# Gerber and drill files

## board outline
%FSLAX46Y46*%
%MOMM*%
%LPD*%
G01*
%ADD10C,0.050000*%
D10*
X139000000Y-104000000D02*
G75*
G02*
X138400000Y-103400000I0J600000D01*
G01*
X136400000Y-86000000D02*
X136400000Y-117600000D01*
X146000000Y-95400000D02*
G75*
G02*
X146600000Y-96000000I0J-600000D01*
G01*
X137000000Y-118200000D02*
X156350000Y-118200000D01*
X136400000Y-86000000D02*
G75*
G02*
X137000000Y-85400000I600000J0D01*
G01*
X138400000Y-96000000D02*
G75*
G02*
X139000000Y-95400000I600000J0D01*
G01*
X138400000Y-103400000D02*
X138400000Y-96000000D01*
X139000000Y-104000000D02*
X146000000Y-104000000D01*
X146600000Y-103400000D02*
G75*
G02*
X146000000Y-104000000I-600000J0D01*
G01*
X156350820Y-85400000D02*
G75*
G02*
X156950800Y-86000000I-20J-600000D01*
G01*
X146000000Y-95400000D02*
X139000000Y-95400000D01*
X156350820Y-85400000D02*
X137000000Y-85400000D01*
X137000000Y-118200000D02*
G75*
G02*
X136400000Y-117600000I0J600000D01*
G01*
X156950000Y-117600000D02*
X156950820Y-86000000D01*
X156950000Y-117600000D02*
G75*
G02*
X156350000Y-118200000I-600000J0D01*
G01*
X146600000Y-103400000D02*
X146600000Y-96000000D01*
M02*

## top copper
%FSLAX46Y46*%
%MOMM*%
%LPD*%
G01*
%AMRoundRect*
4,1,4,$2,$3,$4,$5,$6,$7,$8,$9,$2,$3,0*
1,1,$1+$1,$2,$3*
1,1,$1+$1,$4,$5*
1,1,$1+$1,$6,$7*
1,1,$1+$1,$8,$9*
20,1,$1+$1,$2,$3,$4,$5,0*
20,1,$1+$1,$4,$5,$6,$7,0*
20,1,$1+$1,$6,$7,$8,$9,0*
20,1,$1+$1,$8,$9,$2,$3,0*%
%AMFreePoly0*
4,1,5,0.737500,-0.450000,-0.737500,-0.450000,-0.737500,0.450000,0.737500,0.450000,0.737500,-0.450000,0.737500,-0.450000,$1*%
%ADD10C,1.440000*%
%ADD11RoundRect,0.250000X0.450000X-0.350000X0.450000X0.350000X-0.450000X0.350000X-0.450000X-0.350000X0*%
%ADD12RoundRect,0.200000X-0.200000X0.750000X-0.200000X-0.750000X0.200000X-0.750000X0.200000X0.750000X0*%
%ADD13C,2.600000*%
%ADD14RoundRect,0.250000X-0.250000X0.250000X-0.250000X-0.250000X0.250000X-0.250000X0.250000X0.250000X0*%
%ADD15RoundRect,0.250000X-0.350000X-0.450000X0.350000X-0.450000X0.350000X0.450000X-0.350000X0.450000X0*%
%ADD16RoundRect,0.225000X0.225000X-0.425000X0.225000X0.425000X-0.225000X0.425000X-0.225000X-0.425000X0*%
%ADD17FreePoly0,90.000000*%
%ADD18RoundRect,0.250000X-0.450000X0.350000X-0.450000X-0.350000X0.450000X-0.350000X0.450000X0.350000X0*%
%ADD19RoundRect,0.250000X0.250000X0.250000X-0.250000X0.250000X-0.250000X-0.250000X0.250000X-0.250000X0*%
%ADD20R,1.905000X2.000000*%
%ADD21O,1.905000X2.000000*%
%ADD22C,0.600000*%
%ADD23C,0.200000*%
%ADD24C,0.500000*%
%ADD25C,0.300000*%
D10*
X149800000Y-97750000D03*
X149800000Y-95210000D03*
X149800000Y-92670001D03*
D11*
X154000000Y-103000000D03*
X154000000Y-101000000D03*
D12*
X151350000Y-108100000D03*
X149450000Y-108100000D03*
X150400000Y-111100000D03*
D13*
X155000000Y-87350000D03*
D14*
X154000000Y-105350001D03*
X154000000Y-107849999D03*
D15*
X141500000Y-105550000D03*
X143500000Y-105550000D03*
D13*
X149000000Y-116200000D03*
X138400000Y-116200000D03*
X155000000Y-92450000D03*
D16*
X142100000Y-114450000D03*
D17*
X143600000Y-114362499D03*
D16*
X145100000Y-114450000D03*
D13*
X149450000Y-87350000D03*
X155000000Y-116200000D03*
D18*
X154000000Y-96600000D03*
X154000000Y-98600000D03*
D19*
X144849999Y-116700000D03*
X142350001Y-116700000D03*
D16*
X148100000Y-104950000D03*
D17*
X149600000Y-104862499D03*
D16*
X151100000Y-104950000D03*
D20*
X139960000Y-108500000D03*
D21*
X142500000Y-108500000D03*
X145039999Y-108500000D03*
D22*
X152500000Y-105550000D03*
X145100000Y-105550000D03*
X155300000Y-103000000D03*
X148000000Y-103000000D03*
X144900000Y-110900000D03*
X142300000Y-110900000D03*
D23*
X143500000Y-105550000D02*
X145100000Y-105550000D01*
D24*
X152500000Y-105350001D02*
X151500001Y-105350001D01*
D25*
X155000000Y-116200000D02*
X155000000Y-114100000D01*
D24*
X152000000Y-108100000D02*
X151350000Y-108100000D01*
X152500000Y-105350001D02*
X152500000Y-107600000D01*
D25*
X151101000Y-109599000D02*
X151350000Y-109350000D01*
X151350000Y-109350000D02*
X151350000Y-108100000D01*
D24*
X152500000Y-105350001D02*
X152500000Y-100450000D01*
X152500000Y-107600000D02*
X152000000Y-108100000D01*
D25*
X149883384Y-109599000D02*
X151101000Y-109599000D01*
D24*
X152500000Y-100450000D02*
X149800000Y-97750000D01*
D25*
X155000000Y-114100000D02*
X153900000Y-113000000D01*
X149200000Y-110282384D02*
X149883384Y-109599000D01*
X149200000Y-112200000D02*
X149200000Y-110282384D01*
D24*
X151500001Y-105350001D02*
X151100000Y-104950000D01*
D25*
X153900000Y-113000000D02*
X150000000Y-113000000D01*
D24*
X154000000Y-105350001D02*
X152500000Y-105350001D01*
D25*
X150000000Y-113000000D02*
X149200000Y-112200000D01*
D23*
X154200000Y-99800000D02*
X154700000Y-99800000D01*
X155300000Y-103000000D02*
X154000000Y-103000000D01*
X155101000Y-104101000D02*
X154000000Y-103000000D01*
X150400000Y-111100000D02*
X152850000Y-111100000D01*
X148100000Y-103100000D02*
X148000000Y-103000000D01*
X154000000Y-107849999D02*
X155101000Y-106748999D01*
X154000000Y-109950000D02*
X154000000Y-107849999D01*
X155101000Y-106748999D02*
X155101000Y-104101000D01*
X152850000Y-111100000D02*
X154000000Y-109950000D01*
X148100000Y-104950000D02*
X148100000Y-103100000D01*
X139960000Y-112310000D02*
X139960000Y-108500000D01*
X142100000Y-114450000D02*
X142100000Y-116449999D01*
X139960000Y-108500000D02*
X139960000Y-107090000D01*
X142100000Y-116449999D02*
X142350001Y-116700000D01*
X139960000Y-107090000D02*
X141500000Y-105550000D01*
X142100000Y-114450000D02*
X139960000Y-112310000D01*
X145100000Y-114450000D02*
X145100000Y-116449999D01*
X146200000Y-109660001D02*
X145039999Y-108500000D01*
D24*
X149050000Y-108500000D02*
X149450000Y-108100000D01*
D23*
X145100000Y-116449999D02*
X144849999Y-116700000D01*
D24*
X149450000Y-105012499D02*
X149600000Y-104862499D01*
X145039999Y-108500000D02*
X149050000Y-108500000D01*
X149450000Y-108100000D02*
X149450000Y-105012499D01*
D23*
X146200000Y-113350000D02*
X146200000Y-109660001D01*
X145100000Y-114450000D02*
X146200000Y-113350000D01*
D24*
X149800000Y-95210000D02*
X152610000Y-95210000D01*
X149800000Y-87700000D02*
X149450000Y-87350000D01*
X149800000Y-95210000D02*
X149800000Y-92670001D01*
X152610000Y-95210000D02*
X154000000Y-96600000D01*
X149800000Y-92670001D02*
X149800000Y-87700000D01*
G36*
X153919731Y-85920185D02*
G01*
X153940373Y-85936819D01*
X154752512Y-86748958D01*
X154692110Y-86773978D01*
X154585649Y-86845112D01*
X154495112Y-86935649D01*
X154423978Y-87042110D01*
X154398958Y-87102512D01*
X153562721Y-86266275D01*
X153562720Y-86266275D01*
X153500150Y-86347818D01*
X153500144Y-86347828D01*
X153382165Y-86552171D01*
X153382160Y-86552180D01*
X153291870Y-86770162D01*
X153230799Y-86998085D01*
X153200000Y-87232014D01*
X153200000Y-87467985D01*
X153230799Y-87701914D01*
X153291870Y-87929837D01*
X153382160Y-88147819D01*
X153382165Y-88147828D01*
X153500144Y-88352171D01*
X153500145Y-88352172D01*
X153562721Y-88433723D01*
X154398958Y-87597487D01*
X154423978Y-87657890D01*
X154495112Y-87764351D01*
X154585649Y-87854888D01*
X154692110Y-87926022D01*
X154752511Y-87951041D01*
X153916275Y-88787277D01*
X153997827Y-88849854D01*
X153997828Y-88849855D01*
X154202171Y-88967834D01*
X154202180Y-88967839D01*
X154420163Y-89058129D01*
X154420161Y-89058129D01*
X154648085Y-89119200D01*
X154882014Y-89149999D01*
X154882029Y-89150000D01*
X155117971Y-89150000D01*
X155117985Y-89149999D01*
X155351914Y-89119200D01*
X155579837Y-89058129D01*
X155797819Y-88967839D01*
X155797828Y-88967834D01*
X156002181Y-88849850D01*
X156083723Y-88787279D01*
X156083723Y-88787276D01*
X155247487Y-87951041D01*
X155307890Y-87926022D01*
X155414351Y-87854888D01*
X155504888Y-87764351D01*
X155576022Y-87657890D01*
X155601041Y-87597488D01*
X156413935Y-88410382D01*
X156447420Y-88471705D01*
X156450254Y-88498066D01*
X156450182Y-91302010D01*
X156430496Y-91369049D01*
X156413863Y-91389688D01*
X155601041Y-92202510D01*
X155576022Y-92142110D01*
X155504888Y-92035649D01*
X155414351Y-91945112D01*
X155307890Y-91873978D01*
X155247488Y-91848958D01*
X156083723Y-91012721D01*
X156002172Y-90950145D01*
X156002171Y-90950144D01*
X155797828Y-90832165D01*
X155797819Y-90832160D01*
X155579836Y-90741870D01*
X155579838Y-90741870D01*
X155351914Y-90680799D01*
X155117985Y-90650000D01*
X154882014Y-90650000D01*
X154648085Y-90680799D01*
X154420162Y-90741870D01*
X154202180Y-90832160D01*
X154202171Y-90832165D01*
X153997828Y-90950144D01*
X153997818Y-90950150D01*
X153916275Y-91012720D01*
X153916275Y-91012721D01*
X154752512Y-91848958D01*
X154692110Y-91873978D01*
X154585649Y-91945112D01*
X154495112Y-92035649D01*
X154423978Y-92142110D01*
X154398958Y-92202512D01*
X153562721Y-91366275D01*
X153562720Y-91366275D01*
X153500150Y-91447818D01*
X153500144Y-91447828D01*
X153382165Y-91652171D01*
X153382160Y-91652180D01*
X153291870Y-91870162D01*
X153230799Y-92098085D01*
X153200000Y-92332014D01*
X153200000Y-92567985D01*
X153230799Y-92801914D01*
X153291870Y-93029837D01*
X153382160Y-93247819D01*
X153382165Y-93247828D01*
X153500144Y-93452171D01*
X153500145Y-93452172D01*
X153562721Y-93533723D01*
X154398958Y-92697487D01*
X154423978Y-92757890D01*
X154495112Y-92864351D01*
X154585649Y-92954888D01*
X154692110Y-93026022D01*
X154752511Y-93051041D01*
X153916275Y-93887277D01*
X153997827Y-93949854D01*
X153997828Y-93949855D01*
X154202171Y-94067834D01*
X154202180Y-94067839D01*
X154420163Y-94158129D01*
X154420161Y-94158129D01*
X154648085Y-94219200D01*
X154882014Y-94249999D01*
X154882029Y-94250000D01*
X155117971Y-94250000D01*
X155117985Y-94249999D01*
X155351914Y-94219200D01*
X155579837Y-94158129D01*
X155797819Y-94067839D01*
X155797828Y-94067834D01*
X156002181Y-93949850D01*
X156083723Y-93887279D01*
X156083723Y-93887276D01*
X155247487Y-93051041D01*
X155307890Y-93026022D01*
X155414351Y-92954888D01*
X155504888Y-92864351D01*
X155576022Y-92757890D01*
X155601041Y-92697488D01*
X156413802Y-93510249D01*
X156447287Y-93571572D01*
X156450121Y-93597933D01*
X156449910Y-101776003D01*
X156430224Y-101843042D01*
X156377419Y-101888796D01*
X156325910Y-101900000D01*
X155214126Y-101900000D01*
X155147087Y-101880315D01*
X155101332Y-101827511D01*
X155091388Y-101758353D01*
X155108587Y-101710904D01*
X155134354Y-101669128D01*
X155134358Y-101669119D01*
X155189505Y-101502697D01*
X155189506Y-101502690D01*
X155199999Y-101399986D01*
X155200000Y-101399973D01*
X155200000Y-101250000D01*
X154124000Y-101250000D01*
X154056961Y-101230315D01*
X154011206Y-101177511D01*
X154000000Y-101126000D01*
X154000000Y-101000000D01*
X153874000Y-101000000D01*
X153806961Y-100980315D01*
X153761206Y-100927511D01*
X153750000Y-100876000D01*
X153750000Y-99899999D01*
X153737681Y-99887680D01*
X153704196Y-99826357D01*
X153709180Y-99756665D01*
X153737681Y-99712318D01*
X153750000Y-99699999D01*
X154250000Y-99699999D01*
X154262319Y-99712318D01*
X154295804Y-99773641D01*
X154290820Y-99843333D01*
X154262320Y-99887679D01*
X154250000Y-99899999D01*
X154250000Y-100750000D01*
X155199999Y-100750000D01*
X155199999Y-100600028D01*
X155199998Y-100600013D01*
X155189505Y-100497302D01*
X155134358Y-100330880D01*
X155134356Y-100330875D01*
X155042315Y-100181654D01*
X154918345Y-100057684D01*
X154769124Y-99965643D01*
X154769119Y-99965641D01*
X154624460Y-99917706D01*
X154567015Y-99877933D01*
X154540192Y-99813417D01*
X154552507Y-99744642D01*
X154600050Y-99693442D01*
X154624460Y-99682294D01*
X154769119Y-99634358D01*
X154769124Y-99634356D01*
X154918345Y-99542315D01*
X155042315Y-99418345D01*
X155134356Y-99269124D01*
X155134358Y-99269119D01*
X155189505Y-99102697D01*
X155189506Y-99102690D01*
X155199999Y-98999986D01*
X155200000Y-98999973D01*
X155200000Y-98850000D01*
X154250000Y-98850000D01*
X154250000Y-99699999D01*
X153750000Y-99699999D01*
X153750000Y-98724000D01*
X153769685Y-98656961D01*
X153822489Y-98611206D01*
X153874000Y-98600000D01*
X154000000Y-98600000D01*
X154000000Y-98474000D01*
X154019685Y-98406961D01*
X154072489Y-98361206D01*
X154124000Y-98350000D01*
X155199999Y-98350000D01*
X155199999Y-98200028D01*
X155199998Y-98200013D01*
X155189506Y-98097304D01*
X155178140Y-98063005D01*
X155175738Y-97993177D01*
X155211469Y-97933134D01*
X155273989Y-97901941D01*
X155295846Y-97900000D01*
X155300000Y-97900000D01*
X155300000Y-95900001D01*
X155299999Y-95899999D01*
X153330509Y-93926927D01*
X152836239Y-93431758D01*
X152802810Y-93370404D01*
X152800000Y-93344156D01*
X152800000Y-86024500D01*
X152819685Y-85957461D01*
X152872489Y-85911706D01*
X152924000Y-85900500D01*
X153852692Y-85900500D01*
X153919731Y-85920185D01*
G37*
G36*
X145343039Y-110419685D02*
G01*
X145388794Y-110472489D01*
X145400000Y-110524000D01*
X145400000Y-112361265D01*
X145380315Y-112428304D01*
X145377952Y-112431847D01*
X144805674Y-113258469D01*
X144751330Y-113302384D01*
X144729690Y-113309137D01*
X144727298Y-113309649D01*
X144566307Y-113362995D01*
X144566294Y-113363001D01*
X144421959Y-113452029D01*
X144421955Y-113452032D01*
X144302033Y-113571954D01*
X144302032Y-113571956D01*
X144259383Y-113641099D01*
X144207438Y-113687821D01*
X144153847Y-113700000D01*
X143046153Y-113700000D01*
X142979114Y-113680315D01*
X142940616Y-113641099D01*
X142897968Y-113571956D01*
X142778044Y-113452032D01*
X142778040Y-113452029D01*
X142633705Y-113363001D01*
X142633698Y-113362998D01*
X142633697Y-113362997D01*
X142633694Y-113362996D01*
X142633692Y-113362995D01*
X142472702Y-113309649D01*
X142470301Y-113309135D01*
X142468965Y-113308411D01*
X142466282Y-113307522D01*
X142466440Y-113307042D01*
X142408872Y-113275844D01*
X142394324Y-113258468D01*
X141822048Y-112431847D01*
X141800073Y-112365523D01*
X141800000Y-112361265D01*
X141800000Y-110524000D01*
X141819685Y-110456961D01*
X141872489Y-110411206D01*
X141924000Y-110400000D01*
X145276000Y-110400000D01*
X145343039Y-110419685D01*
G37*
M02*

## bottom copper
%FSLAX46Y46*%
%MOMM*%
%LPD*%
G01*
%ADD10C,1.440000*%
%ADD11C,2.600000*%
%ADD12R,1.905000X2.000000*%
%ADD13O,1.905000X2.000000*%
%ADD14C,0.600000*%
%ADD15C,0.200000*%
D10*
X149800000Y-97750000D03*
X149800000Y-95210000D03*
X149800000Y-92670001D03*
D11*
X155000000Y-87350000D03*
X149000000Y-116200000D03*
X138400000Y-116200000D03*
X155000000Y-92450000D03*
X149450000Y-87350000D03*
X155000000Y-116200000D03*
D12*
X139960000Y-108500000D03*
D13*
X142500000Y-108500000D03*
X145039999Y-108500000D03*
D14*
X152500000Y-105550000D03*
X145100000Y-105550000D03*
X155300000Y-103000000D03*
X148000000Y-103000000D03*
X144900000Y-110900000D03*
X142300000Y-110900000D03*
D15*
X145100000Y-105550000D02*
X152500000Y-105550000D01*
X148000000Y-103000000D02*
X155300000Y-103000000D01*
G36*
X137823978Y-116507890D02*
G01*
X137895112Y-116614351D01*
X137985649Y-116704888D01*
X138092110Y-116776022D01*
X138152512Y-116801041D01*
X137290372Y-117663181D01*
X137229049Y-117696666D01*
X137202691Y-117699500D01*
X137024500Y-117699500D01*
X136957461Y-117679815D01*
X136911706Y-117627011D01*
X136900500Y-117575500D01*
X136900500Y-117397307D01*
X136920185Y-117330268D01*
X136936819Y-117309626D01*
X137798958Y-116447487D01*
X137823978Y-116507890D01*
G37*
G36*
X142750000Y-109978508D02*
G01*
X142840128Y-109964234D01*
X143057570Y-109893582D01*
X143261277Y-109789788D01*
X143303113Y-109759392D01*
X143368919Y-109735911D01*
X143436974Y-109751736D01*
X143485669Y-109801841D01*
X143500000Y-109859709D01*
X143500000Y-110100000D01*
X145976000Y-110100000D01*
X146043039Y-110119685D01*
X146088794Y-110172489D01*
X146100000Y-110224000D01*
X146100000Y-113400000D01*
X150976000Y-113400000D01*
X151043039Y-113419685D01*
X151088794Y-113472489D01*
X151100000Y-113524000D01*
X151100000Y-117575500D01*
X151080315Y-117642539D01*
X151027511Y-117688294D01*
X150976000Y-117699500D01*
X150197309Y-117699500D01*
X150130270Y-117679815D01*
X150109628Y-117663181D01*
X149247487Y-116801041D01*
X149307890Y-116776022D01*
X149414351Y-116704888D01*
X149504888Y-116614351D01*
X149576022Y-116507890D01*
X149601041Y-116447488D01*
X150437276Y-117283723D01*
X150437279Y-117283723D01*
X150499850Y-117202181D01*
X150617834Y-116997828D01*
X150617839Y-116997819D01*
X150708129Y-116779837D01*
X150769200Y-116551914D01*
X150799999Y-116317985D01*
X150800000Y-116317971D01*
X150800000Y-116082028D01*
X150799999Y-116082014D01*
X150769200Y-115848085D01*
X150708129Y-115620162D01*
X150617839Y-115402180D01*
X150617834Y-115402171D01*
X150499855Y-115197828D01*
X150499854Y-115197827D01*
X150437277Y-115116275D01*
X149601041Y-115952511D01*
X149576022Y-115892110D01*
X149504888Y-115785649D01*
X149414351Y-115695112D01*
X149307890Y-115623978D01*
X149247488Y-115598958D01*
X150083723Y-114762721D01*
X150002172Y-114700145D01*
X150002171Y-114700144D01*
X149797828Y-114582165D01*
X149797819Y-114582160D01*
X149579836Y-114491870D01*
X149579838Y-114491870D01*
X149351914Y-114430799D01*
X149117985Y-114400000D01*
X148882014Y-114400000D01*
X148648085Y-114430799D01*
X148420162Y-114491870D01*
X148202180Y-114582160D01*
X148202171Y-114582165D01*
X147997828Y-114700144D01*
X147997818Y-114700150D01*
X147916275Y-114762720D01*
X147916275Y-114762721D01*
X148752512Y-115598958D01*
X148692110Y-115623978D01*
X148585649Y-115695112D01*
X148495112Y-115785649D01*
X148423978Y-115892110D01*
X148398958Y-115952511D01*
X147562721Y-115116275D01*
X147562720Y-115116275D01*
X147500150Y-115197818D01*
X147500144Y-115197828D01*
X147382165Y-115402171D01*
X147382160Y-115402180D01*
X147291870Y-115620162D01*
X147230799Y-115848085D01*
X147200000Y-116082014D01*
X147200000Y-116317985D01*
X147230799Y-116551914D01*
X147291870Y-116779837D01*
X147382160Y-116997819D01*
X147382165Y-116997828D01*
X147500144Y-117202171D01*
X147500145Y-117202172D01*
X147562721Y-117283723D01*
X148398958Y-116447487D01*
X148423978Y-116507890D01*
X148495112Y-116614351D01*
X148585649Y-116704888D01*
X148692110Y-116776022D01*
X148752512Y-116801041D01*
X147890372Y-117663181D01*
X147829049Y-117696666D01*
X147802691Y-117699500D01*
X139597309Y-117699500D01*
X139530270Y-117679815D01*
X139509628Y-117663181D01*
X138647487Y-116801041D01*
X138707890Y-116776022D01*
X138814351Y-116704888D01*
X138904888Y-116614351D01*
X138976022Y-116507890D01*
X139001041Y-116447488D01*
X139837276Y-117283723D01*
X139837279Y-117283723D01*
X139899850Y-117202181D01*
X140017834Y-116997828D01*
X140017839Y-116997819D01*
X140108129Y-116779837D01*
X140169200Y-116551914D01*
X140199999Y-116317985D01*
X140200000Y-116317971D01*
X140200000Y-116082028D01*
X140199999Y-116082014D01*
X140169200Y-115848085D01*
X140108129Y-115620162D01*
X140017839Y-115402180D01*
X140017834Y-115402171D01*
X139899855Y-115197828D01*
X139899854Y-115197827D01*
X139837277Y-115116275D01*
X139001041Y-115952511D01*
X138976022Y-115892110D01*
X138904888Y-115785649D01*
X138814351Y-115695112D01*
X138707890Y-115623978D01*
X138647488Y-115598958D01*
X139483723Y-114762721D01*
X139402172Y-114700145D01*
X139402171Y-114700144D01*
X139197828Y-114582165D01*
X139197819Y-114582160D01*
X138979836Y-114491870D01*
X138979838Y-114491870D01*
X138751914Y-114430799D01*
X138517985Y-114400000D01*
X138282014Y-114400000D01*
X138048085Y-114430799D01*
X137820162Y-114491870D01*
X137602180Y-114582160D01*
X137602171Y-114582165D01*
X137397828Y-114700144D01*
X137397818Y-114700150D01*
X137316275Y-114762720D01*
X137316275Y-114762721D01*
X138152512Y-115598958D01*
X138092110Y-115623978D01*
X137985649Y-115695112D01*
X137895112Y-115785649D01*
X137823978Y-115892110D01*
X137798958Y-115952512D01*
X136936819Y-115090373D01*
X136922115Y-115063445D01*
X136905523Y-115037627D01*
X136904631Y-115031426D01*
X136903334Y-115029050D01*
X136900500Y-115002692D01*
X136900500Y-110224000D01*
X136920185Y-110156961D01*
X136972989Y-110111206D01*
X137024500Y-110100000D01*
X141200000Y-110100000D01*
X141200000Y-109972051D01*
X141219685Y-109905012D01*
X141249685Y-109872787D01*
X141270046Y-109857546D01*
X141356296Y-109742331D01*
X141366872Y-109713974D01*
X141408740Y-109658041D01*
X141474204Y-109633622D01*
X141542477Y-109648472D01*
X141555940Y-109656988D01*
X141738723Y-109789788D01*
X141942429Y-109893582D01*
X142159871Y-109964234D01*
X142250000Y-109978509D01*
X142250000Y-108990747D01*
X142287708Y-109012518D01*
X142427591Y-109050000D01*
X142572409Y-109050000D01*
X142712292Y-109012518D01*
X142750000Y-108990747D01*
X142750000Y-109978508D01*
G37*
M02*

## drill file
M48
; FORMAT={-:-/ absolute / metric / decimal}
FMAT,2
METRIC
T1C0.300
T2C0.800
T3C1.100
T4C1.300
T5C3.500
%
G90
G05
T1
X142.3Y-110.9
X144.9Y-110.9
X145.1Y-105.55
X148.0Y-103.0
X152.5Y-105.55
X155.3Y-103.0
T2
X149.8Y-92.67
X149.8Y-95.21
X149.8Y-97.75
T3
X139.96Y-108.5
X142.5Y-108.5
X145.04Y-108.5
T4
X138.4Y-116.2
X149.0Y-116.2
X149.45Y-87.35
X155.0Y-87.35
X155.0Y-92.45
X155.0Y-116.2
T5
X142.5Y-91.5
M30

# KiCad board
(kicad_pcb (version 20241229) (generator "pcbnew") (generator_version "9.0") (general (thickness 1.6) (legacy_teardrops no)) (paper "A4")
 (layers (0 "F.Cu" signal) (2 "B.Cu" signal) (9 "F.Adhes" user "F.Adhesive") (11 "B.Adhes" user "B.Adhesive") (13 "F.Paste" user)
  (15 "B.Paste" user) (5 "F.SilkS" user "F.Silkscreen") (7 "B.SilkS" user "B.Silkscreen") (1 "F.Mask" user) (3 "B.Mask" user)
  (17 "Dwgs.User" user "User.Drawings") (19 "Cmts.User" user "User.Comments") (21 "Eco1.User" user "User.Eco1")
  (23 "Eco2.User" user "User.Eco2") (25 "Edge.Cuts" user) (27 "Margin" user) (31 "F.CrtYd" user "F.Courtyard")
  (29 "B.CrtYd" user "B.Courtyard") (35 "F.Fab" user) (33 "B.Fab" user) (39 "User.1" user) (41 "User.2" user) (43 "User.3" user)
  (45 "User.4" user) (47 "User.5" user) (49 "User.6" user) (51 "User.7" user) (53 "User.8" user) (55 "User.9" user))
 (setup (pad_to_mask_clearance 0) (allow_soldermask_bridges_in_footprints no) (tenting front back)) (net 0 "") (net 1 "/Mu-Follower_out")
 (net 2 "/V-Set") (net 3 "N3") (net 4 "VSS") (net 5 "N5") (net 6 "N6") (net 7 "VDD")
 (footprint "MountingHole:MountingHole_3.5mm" (layer "F.Cu") (at 142.5 91.5)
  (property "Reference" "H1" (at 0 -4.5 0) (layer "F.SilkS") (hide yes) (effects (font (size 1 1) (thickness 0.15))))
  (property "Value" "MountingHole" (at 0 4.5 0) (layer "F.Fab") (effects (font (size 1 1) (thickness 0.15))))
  (pad "" np_thru_hole circle (at 0 0) (size 3.5 3.5) (drill 3.5) (layers "*.Cu" "*.Mask")))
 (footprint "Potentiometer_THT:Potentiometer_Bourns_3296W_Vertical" (layer "F.Cu") (at 149.8 97.75 -90)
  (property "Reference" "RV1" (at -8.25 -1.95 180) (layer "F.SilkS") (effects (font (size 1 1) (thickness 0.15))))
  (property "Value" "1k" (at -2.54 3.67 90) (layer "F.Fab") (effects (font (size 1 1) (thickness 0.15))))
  (pad "1" thru_hole circle (at 0 0 270) (size 1.44 1.44) (drill 0.8) (layers "*.Cu" "*.Mask") (remove_unused_layers no)
   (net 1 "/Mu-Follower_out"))
  (pad "2" thru_hole circle (at -2.54 0 270) (size 1.44 1.44) (drill 0.8) (layers "*.Cu" "*.Mask") (remove_unused_layers no)
   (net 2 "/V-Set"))
  (pad "3" thru_hole circle (at -5.079999 0 270) (size 1.44 1.44) (drill 0.8) (layers "*.Cu" "*.Mask") (remove_unused_layers no)
   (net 2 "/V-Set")))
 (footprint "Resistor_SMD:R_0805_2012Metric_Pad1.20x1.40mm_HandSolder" (layer "F.Cu") (at 154 102 90)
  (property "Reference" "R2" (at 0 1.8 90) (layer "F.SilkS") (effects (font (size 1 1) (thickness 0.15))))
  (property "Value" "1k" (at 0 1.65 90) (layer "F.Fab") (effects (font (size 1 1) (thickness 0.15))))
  (pad "1" smd roundrect (at -1 0 90) (size 1.2 1.4) (layers "F.Cu" "F.Mask" "F.Paste") (roundrect_rratio 0.208333) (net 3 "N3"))
  (pad "2" smd roundrect (at 1 0 90) (size 1.2 1.4) (layers "F.Cu" "F.Mask" "F.Paste") (roundrect_rratio 0.208333) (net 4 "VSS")))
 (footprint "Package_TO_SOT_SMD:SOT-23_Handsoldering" (layer "F.Cu") (at 150.4 109.6 -90)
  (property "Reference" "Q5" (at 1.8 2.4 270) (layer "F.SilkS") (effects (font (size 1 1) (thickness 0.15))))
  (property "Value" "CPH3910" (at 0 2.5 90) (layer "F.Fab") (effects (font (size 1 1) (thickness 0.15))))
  (pad "1" smd roundrect (at -1.5 -0.95 270) (size 1.9 0.8) (layers "F.Cu" "F.Mask" "F.Paste") (roundrect_rratio 0.25)
   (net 1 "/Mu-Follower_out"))
  (pad "2" smd roundrect (at -1.5 0.95 270) (size 1.9 0.8) (layers "F.Cu" "F.Mask" "F.Paste") (roundrect_rratio 0.25) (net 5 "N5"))
  (pad "3" smd roundrect (at 1.5 0 270) (size 1.9 0.8) (layers "F.Cu" "F.Mask" "F.Paste") (roundrect_rratio 0.25) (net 3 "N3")))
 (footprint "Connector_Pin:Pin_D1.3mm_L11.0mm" (layer "F.Cu") (at 155 87.35 180)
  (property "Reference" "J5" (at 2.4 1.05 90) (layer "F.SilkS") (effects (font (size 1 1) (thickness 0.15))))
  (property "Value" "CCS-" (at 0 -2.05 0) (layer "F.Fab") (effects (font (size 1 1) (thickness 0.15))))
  (pad "1" thru_hole circle (at 0 0 180) (size 2.6 2.6) (drill 1.3) (layers "*.Cu" "*.Mask") (remove_unused_layers no) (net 4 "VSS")))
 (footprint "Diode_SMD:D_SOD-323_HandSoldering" (layer "F.Cu") (at 154 106.6 -90)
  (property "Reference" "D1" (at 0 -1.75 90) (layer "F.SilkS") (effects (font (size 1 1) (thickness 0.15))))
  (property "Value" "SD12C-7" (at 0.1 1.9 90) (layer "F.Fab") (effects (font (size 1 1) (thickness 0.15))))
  (pad "1" smd roundrect (at -1.249999 0 270) (size 1 1) (layers "F.Cu" "F.Mask" "F.Paste") (roundrect_rratio 0.25)
   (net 1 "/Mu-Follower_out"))
  (pad "2" smd roundrect (at 1.249999 0 270) (size 1 1) (layers "F.Cu" "F.Mask" "F.Paste") (roundrect_rratio 0.25) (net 3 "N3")))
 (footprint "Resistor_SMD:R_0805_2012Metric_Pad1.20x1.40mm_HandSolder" (layer "F.Cu") (at 142.5 105.55)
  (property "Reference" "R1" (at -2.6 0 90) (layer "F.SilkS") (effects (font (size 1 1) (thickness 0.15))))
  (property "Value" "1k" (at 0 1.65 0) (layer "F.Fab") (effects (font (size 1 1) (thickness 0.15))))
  (pad "1" smd roundrect (at -1 0) (size 1.2 1.4) (layers "F.Cu" "F.Mask" "F.Paste") (roundrect_rratio 0.208333) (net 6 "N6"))
  (pad "2" smd roundrect (at 1 0) (size 1.2 1.4) (layers "F.Cu" "F.Mask" "F.Paste") (roundrect_rratio 0.208333) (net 1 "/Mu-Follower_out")))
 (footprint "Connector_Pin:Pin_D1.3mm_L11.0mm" (layer "F.Cu") (at 149 116.2)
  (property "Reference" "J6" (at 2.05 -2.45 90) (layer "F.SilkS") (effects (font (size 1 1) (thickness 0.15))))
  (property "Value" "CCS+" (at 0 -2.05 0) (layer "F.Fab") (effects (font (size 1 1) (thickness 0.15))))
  (pad "1" thru_hole circle (at 0 0) (size 2.6 2.6) (drill 1.3) (layers "*.Cu" "*.Mask") (remove_unused_layers no) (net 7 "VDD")))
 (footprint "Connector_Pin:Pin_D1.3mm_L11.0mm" (layer "F.Cu") (at 138.4 116.2)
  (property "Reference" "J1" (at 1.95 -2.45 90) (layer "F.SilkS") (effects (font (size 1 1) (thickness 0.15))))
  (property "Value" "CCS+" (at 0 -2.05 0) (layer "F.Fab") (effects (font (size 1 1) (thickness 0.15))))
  (pad "1" thru_hole circle (at 0 0) (size 2.6 2.6) (drill 1.3) (layers "*.Cu" "*.Mask") (remove_unused_layers no) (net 7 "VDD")))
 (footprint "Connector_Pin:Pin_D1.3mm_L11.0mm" (layer "F.Cu") (at 155 92.45 180)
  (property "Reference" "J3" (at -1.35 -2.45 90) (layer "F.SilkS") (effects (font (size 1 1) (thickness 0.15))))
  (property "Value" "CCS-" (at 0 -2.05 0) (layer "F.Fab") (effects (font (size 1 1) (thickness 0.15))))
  (pad "1" thru_hole circle (at 0 0 180) (size 2.6 2.6) (drill 1.3) (layers "*.Cu" "*.Mask") (remove_unused_layers no) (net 4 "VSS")))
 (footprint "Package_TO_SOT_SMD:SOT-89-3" (layer "F.Cu") (at 143.6 112.5 90)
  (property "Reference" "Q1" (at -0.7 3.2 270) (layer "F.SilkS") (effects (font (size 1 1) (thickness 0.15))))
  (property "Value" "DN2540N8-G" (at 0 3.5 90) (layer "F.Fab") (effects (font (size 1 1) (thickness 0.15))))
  (pad "1" smd roundrect (at -1.95 -1.5 90) (size 1.3 0.9) (layers "F.Cu" "F.Mask" "F.Paste") (roundrect_rratio 0.25) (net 6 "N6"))
  (pad "2" smd custom (at -1.862499 0 90) (size 1.475 0.9) (layers "F.Cu" "F.Mask" "F.Paste") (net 7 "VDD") (zone_connect 2)
   (thermal_bridge_angle 45) (options (clearance outline) (anchor rect)) (primitives))
  (pad "3" smd roundrect (at -1.95 1.5 90) (size 1.3 0.9) (layers "F.Cu" "F.Mask" "F.Paste") (roundrect_rratio 0.25) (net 5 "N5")))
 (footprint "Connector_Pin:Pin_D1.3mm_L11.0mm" (layer "F.Cu") (at 149.45 87.35 180)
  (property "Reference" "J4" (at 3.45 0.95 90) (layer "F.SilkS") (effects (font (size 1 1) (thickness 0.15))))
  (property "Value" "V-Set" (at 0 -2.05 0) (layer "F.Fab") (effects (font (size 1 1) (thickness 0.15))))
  (pad "1" thru_hole circle (at 0 0 180) (size 2.6 2.6) (drill 1.3) (layers "*.Cu" "*.Mask") (remove_unused_layers no) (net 2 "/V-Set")))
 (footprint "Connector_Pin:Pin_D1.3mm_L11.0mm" (layer "F.Cu") (at 155 116.2)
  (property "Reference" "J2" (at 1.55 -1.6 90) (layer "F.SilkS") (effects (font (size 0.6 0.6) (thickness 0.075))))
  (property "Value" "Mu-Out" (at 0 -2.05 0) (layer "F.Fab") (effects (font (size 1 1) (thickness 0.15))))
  (pad "1" thru_hole circle (at 0 0) (size 2.6 2.6) (drill 1.3) (layers "*.Cu" "*.Mask") (remove_unused_layers no)
   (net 1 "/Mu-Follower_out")))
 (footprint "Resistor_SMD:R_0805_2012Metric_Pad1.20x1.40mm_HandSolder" (layer "F.Cu") (at 154 97.6 -90)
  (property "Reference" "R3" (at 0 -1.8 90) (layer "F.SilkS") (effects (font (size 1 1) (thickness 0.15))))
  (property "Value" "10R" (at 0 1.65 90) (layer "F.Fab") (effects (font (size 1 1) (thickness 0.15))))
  (pad "1" smd roundrect (at -1 0 270) (size 1.2 1.4) (layers "F.Cu" "F.Mask" "F.Paste") (roundrect_rratio 0.208333) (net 2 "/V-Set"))
  (pad "2" smd roundrect (at 1 0 270) (size 1.2 1.4) (layers "F.Cu" "F.Mask" "F.Paste") (roundrect_rratio 0.208333) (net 4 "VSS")))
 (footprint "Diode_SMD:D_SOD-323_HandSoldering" (layer "F.Cu") (at 143.6 116.7 180)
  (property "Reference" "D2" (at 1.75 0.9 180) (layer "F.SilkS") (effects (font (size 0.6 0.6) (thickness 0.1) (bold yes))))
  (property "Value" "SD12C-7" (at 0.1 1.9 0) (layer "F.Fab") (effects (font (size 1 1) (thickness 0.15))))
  (pad "1" smd roundrect (at -1.249999 0 180) (size 1 1) (layers "F.Cu" "F.Mask" "F.Paste") (roundrect_rratio 0.25) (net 5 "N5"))
  (pad "2" smd roundrect (at 1.249999 0 180) (size 1 1) (layers "F.Cu" "F.Mask" "F.Paste") (roundrect_rratio 0.25) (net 6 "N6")))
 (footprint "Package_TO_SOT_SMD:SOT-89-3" (layer "F.Cu") (at 149.6 103 90)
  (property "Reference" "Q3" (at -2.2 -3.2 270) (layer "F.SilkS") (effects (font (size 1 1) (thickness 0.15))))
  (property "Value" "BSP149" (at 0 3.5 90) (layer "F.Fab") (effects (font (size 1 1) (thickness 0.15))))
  (pad "1" smd roundrect (at -1.95 -1.5 90) (size 1.3 0.9) (layers "F.Cu" "F.Mask" "F.Paste") (roundrect_rratio 0.25) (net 3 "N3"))
  (pad "2" smd custom (at -1.862499 0 90) (size 1.475 0.9) (layers "F.Cu" "F.Mask" "F.Paste") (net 5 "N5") (zone_connect 2)
   (thermal_bridge_angle 45) (options (clearance outline) (anchor rect)) (primitives))
  (pad "3" smd roundrect (at -1.95 1.5 90) (size 1.3 0.9) (layers "F.Cu" "F.Mask" "F.Paste") (roundrect_rratio 0.25)
   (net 1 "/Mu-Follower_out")))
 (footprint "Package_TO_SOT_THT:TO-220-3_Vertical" (layer "B.Cu") (at 139.96 108.5)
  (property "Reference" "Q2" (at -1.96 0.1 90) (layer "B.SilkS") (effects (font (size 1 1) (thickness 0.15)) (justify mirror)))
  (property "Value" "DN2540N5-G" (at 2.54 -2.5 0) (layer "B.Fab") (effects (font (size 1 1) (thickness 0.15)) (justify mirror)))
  (pad "1" thru_hole rect (at 0 0) (size 1.905 2) (drill 1.1) (layers "*.Cu" "*.Mask") (remove_unused_layers no) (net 6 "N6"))
  (pad "2" thru_hole oval (at 2.54 0) (size 1.905 2) (drill 1.1) (layers "*.Cu" "*.Mask") (remove_unused_layers no) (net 7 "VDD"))
  (pad "3" thru_hole oval (at 5.079999 0) (size 1.905 2) (drill 1.1) (layers "*.Cu" "*.Mask") (remove_unused_layers no) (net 5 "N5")))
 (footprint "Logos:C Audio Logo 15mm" (layer "B.Cu") (at 152 111.6)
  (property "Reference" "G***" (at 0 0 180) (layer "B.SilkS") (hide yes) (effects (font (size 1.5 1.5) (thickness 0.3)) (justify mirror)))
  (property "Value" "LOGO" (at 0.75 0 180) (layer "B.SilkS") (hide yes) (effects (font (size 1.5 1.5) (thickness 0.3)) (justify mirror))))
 (gr_arc (start 139 104) (mid 138.575736 103.824264) (end 138.4 103.4) (stroke (width 0.05) (type default)) (layer "Edge.Cuts"))
 (gr_line (start 136.4 86) (end 136.4 117.6) (stroke (width 0.05) (type default)) (layer "Edge.Cuts"))
 (gr_arc (start 146 95.4) (mid 146.424264 95.575736) (end 146.6 96) (stroke (width 0.05) (type default)) (layer "Edge.Cuts"))
 (gr_line (start 137 118.2) (end 156.35 118.2) (stroke (width 0.05) (type default)) (layer "Edge.Cuts"))
 (gr_arc (start 136.4 86) (mid 136.575736 85.575736) (end 137 85.4) (stroke (width 0.05) (type default)) (layer "Edge.Cuts"))
 (gr_arc (start 138.4 96) (mid 138.575736 95.575736) (end 139 95.4) (stroke (width 0.05) (type default)) (layer "Edge.Cuts"))
 (gr_line (start 138.4 103.4) (end 138.4 96) (stroke (width 0.05) (type default)) (layer "Edge.Cuts"))
 (gr_line (start 139 104) (end 146 104) (stroke (width 0.05) (type default)) (layer "Edge.Cuts"))
 (gr_arc (start 146.6 103.4) (mid 146.424264 103.824264) (end 146 104) (stroke (width 0.05) (type default)) (layer "Edge.Cuts"))
 (gr_arc (start 156.35082 85.4) (mid 156.775084 85.575736) (end 156.95082 86) (stroke (width 0.05) (type default)) (layer "Edge.Cuts"))
 (gr_line (start 146 95.4) (end 139 95.4) (stroke (width 0.05) (type default)) (layer "Edge.Cuts"))
 (gr_line (start 156.35082 85.4) (end 137 85.4) (stroke (width 0.05) (type default)) (layer "Edge.Cuts"))
 (gr_arc (start 137 118.2) (mid 136.575736 118.024264) (end 136.4 117.6) (stroke (width 0.05) (type default)) (layer "Edge.Cuts"))
 (gr_line (start 156.95 117.6) (end 156.95082 86) (stroke (width 0.05) (type default)) (layer "Edge.Cuts"))
 (gr_arc (start 156.95 117.6) (mid 156.774264 118.024264) (end 156.35 118.2) (stroke (width 0.05) (type default)) (layer "Edge.Cuts"))
 (gr_line (start 146.6 103.4) (end 146.6 96) (stroke (width 0.05) (type default)) (layer "Edge.Cuts"))
 (segment (start 143.5 105.55) (end 145.1 105.55) (width 0.2) (layer "F.Cu") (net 1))
 (segment (start 152.5 105.350001) (end 151.500001 105.350001) (width 0.5) (layer "F.Cu") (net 1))
 (segment (start 155 116.2) (end 155 114.1) (width 0.3) (layer "F.Cu") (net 1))
 (segment (start 152 108.1) (end 151.35 108.1) (width 0.5) (layer "F.Cu") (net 1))
 (segment (start 152.5 105.350001) (end 152.5 107.6) (width 0.5) (layer "F.Cu") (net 1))
 (segment (start 151.101 109.599) (end 151.35 109.35) (width 0.3) (layer "F.Cu") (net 1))
 (segment (start 151.35 109.35) (end 151.35 108.1) (width 0.3) (layer "F.Cu") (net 1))
 (segment (start 152.5 105.350001) (end 152.5 100.45) (width 0.5) (layer "F.Cu") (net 1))
 (segment (start 152.5 107.6) (end 152 108.1) (width 0.5) (layer "F.Cu") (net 1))
 (segment (start 149.883384 109.599) (end 151.101 109.599) (width 0.3) (layer "F.Cu") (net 1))
 (segment (start 152.5 100.45) (end 149.8 97.75) (width 0.5) (layer "F.Cu") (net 1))
 (segment (start 155 114.1) (end 153.9 113) (width 0.3) (layer "F.Cu") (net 1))
 (segment (start 149.2 110.282384) (end 149.883384 109.599) (width 0.3) (layer "F.Cu") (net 1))
 (segment (start 149.2 112.2) (end 149.2 110.282384) (width 0.3) (layer "F.Cu") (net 1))
 (segment (start 151.500001 105.350001) (end 151.1 104.95) (width 0.5) (layer "F.Cu") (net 1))
 (segment (start 153.9 113) (end 150 113) (width 0.3) (layer "F.Cu") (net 1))
 (segment (start 154 105.350001) (end 152.5 105.350001) (width 0.5) (layer "F.Cu") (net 1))
 (segment (start 150 113) (end 149.2 112.2) (width 0.3) (layer "F.Cu") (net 1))
 (via (at 152.5 105.55) (size 0.6) (drill 0.3) (layers "F.Cu" "B.Cu") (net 1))
 (via (at 145.1 105.55) (size 0.6) (drill 0.3) (layers "F.Cu" "B.Cu") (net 1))
 (segment (start 145.1 105.55) (end 152.5 105.55) (width 0.2) (layer "B.Cu") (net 1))
 (segment (start 154.2 99.8) (end 154.7 99.8) (width 0.2) (layer "F.Cu") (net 4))
 (segment (start 155.3 103) (end 154 103) (width 0.2) (layer "F.Cu") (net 3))
 (segment (start 155.101 104.101) (end 154 103) (width 0.2) (layer "F.Cu") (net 3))
 (segment (start 150.4 111.1) (end 152.85 111.1) (width 0.2) (layer "F.Cu") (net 3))
 (segment (start 148.1 103.1) (end 148 103) (width 0.2) (layer "F.Cu") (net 3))
 (segment (start 154 107.849999) (end 155.101 106.748999) (width 0.2) (layer "F.Cu") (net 3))
 (segment (start 154 109.95) (end 154 107.849999) (width 0.2) (layer "F.Cu") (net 3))
 (segment (start 155.101 106.748999) (end 155.101 104.101) (width 0.2) (layer "F.Cu") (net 3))
 (segment (start 152.85 111.1) (end 154 109.95) (width 0.2) (layer "F.Cu") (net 3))
 (segment (start 148.1 104.95) (end 148.1 103.1) (width 0.2) (layer "F.Cu") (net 3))
 (via (at 155.3 103) (size 0.6) (drill 0.3) (layers "F.Cu" "B.Cu") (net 3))
 (via (at 148 103) (size 0.6) (drill 0.3) (layers "F.Cu" "B.Cu") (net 3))
 (segment (start 148 103) (end 155.3 103) (width 0.2) (layer "B.Cu") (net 3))
 (segment (start 139.96 112.31) (end 139.96 108.5) (width 0.2) (layer "F.Cu") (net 6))
 (segment (start 142.1 114.45) (end 142.1 116.449999) (width 0.2) (layer "F.Cu") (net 6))
 (segment (start 139.96 108.5) (end 139.96 107.09) (width 0.2) (layer "F.Cu") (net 6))
 (segment (start 142.1 116.449999) (end 142.350001 116.7) (width 0.2) (layer "F.Cu") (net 6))
 (segment (start 139.96 107.09) (end 141.5 105.55) (width 0.2) (layer "F.Cu") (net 6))
 (segment (start 142.1 114.45) (end 139.96 112.31) (width 0.2) (layer "F.Cu") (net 6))
 (segment (start 145.1 114.45) (end 145.1 116.449999) (width 0.2) (layer "F.Cu") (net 5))
 (segment (start 146.2 109.660001) (end 145.039999 108.5) (width 0.2) (layer "F.Cu") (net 5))
 (segment (start 149.05 108.5) (end 149.45 108.1) (width 0.5) (layer "F.Cu") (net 5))
 (segment (start 145.1 116.449999) (end 144.849999 116.7) (width 0.2) (layer "F.Cu") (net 5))
 (segment (start 149.45 105.012499) (end 149.6 104.862499) (width 0.5) (layer "F.Cu") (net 5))
 (segment (start 145.039999 108.5) (end 149.05 108.5) (width 0.5) (layer "F.Cu") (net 5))
 (segment (start 149.45 108.1) (end 149.45 105.012499) (width 0.5) (layer "F.Cu") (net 5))
 (segment (start 146.2 113.35) (end 146.2 109.660001) (width 0.2) (layer "F.Cu") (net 5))
 (segment (start 145.1 114.45) (end 146.2 113.35) (width 0.2) (layer "F.Cu") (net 5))
 (segment (start 149.8 95.21) (end 152.61 95.21) (width 0.5) (layer "F.Cu") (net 2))
 (segment (start 149.8 87.7) (end 149.45 87.35) (width 0.5) (layer "F.Cu") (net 2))
 (segment (start 149.8 95.21) (end 149.8 92.670001) (width 0.5) (layer "F.Cu") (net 2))
 (segment (start 152.61 95.21) (end 154 96.6) (width 0.5) (layer "F.Cu") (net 2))
 (segment (start 149.8 92.670001) (end 149.8 87.7) (width 0.5) (layer "F.Cu") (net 2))
 (via (at 144.9 110.9) (size 0.6) (drill 0.3) (layers "F.Cu" "B.Cu") (free yes) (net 7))
 (via (at 142.3 110.9) (size 0.6) (drill 0.3) (layers "F.Cu" "B.Cu") (free yes) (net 7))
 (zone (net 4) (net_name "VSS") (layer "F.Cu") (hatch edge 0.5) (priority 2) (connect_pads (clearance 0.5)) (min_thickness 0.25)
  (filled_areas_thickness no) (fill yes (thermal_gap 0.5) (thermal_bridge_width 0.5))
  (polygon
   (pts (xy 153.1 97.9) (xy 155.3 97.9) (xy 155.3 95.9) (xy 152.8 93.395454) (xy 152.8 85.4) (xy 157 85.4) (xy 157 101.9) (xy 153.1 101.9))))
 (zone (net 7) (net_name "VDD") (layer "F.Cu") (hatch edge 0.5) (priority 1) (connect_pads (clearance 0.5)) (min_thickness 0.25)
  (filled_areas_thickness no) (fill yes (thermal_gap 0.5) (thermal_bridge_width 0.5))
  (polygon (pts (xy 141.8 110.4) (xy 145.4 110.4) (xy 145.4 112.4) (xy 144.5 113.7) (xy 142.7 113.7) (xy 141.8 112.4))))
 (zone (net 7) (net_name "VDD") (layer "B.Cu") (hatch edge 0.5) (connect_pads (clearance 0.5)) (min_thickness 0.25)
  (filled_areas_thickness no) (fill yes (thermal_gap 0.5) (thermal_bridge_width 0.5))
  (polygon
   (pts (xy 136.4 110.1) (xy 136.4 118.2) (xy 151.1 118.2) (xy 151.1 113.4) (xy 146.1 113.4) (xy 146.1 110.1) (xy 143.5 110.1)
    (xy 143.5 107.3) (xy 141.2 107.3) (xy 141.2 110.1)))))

